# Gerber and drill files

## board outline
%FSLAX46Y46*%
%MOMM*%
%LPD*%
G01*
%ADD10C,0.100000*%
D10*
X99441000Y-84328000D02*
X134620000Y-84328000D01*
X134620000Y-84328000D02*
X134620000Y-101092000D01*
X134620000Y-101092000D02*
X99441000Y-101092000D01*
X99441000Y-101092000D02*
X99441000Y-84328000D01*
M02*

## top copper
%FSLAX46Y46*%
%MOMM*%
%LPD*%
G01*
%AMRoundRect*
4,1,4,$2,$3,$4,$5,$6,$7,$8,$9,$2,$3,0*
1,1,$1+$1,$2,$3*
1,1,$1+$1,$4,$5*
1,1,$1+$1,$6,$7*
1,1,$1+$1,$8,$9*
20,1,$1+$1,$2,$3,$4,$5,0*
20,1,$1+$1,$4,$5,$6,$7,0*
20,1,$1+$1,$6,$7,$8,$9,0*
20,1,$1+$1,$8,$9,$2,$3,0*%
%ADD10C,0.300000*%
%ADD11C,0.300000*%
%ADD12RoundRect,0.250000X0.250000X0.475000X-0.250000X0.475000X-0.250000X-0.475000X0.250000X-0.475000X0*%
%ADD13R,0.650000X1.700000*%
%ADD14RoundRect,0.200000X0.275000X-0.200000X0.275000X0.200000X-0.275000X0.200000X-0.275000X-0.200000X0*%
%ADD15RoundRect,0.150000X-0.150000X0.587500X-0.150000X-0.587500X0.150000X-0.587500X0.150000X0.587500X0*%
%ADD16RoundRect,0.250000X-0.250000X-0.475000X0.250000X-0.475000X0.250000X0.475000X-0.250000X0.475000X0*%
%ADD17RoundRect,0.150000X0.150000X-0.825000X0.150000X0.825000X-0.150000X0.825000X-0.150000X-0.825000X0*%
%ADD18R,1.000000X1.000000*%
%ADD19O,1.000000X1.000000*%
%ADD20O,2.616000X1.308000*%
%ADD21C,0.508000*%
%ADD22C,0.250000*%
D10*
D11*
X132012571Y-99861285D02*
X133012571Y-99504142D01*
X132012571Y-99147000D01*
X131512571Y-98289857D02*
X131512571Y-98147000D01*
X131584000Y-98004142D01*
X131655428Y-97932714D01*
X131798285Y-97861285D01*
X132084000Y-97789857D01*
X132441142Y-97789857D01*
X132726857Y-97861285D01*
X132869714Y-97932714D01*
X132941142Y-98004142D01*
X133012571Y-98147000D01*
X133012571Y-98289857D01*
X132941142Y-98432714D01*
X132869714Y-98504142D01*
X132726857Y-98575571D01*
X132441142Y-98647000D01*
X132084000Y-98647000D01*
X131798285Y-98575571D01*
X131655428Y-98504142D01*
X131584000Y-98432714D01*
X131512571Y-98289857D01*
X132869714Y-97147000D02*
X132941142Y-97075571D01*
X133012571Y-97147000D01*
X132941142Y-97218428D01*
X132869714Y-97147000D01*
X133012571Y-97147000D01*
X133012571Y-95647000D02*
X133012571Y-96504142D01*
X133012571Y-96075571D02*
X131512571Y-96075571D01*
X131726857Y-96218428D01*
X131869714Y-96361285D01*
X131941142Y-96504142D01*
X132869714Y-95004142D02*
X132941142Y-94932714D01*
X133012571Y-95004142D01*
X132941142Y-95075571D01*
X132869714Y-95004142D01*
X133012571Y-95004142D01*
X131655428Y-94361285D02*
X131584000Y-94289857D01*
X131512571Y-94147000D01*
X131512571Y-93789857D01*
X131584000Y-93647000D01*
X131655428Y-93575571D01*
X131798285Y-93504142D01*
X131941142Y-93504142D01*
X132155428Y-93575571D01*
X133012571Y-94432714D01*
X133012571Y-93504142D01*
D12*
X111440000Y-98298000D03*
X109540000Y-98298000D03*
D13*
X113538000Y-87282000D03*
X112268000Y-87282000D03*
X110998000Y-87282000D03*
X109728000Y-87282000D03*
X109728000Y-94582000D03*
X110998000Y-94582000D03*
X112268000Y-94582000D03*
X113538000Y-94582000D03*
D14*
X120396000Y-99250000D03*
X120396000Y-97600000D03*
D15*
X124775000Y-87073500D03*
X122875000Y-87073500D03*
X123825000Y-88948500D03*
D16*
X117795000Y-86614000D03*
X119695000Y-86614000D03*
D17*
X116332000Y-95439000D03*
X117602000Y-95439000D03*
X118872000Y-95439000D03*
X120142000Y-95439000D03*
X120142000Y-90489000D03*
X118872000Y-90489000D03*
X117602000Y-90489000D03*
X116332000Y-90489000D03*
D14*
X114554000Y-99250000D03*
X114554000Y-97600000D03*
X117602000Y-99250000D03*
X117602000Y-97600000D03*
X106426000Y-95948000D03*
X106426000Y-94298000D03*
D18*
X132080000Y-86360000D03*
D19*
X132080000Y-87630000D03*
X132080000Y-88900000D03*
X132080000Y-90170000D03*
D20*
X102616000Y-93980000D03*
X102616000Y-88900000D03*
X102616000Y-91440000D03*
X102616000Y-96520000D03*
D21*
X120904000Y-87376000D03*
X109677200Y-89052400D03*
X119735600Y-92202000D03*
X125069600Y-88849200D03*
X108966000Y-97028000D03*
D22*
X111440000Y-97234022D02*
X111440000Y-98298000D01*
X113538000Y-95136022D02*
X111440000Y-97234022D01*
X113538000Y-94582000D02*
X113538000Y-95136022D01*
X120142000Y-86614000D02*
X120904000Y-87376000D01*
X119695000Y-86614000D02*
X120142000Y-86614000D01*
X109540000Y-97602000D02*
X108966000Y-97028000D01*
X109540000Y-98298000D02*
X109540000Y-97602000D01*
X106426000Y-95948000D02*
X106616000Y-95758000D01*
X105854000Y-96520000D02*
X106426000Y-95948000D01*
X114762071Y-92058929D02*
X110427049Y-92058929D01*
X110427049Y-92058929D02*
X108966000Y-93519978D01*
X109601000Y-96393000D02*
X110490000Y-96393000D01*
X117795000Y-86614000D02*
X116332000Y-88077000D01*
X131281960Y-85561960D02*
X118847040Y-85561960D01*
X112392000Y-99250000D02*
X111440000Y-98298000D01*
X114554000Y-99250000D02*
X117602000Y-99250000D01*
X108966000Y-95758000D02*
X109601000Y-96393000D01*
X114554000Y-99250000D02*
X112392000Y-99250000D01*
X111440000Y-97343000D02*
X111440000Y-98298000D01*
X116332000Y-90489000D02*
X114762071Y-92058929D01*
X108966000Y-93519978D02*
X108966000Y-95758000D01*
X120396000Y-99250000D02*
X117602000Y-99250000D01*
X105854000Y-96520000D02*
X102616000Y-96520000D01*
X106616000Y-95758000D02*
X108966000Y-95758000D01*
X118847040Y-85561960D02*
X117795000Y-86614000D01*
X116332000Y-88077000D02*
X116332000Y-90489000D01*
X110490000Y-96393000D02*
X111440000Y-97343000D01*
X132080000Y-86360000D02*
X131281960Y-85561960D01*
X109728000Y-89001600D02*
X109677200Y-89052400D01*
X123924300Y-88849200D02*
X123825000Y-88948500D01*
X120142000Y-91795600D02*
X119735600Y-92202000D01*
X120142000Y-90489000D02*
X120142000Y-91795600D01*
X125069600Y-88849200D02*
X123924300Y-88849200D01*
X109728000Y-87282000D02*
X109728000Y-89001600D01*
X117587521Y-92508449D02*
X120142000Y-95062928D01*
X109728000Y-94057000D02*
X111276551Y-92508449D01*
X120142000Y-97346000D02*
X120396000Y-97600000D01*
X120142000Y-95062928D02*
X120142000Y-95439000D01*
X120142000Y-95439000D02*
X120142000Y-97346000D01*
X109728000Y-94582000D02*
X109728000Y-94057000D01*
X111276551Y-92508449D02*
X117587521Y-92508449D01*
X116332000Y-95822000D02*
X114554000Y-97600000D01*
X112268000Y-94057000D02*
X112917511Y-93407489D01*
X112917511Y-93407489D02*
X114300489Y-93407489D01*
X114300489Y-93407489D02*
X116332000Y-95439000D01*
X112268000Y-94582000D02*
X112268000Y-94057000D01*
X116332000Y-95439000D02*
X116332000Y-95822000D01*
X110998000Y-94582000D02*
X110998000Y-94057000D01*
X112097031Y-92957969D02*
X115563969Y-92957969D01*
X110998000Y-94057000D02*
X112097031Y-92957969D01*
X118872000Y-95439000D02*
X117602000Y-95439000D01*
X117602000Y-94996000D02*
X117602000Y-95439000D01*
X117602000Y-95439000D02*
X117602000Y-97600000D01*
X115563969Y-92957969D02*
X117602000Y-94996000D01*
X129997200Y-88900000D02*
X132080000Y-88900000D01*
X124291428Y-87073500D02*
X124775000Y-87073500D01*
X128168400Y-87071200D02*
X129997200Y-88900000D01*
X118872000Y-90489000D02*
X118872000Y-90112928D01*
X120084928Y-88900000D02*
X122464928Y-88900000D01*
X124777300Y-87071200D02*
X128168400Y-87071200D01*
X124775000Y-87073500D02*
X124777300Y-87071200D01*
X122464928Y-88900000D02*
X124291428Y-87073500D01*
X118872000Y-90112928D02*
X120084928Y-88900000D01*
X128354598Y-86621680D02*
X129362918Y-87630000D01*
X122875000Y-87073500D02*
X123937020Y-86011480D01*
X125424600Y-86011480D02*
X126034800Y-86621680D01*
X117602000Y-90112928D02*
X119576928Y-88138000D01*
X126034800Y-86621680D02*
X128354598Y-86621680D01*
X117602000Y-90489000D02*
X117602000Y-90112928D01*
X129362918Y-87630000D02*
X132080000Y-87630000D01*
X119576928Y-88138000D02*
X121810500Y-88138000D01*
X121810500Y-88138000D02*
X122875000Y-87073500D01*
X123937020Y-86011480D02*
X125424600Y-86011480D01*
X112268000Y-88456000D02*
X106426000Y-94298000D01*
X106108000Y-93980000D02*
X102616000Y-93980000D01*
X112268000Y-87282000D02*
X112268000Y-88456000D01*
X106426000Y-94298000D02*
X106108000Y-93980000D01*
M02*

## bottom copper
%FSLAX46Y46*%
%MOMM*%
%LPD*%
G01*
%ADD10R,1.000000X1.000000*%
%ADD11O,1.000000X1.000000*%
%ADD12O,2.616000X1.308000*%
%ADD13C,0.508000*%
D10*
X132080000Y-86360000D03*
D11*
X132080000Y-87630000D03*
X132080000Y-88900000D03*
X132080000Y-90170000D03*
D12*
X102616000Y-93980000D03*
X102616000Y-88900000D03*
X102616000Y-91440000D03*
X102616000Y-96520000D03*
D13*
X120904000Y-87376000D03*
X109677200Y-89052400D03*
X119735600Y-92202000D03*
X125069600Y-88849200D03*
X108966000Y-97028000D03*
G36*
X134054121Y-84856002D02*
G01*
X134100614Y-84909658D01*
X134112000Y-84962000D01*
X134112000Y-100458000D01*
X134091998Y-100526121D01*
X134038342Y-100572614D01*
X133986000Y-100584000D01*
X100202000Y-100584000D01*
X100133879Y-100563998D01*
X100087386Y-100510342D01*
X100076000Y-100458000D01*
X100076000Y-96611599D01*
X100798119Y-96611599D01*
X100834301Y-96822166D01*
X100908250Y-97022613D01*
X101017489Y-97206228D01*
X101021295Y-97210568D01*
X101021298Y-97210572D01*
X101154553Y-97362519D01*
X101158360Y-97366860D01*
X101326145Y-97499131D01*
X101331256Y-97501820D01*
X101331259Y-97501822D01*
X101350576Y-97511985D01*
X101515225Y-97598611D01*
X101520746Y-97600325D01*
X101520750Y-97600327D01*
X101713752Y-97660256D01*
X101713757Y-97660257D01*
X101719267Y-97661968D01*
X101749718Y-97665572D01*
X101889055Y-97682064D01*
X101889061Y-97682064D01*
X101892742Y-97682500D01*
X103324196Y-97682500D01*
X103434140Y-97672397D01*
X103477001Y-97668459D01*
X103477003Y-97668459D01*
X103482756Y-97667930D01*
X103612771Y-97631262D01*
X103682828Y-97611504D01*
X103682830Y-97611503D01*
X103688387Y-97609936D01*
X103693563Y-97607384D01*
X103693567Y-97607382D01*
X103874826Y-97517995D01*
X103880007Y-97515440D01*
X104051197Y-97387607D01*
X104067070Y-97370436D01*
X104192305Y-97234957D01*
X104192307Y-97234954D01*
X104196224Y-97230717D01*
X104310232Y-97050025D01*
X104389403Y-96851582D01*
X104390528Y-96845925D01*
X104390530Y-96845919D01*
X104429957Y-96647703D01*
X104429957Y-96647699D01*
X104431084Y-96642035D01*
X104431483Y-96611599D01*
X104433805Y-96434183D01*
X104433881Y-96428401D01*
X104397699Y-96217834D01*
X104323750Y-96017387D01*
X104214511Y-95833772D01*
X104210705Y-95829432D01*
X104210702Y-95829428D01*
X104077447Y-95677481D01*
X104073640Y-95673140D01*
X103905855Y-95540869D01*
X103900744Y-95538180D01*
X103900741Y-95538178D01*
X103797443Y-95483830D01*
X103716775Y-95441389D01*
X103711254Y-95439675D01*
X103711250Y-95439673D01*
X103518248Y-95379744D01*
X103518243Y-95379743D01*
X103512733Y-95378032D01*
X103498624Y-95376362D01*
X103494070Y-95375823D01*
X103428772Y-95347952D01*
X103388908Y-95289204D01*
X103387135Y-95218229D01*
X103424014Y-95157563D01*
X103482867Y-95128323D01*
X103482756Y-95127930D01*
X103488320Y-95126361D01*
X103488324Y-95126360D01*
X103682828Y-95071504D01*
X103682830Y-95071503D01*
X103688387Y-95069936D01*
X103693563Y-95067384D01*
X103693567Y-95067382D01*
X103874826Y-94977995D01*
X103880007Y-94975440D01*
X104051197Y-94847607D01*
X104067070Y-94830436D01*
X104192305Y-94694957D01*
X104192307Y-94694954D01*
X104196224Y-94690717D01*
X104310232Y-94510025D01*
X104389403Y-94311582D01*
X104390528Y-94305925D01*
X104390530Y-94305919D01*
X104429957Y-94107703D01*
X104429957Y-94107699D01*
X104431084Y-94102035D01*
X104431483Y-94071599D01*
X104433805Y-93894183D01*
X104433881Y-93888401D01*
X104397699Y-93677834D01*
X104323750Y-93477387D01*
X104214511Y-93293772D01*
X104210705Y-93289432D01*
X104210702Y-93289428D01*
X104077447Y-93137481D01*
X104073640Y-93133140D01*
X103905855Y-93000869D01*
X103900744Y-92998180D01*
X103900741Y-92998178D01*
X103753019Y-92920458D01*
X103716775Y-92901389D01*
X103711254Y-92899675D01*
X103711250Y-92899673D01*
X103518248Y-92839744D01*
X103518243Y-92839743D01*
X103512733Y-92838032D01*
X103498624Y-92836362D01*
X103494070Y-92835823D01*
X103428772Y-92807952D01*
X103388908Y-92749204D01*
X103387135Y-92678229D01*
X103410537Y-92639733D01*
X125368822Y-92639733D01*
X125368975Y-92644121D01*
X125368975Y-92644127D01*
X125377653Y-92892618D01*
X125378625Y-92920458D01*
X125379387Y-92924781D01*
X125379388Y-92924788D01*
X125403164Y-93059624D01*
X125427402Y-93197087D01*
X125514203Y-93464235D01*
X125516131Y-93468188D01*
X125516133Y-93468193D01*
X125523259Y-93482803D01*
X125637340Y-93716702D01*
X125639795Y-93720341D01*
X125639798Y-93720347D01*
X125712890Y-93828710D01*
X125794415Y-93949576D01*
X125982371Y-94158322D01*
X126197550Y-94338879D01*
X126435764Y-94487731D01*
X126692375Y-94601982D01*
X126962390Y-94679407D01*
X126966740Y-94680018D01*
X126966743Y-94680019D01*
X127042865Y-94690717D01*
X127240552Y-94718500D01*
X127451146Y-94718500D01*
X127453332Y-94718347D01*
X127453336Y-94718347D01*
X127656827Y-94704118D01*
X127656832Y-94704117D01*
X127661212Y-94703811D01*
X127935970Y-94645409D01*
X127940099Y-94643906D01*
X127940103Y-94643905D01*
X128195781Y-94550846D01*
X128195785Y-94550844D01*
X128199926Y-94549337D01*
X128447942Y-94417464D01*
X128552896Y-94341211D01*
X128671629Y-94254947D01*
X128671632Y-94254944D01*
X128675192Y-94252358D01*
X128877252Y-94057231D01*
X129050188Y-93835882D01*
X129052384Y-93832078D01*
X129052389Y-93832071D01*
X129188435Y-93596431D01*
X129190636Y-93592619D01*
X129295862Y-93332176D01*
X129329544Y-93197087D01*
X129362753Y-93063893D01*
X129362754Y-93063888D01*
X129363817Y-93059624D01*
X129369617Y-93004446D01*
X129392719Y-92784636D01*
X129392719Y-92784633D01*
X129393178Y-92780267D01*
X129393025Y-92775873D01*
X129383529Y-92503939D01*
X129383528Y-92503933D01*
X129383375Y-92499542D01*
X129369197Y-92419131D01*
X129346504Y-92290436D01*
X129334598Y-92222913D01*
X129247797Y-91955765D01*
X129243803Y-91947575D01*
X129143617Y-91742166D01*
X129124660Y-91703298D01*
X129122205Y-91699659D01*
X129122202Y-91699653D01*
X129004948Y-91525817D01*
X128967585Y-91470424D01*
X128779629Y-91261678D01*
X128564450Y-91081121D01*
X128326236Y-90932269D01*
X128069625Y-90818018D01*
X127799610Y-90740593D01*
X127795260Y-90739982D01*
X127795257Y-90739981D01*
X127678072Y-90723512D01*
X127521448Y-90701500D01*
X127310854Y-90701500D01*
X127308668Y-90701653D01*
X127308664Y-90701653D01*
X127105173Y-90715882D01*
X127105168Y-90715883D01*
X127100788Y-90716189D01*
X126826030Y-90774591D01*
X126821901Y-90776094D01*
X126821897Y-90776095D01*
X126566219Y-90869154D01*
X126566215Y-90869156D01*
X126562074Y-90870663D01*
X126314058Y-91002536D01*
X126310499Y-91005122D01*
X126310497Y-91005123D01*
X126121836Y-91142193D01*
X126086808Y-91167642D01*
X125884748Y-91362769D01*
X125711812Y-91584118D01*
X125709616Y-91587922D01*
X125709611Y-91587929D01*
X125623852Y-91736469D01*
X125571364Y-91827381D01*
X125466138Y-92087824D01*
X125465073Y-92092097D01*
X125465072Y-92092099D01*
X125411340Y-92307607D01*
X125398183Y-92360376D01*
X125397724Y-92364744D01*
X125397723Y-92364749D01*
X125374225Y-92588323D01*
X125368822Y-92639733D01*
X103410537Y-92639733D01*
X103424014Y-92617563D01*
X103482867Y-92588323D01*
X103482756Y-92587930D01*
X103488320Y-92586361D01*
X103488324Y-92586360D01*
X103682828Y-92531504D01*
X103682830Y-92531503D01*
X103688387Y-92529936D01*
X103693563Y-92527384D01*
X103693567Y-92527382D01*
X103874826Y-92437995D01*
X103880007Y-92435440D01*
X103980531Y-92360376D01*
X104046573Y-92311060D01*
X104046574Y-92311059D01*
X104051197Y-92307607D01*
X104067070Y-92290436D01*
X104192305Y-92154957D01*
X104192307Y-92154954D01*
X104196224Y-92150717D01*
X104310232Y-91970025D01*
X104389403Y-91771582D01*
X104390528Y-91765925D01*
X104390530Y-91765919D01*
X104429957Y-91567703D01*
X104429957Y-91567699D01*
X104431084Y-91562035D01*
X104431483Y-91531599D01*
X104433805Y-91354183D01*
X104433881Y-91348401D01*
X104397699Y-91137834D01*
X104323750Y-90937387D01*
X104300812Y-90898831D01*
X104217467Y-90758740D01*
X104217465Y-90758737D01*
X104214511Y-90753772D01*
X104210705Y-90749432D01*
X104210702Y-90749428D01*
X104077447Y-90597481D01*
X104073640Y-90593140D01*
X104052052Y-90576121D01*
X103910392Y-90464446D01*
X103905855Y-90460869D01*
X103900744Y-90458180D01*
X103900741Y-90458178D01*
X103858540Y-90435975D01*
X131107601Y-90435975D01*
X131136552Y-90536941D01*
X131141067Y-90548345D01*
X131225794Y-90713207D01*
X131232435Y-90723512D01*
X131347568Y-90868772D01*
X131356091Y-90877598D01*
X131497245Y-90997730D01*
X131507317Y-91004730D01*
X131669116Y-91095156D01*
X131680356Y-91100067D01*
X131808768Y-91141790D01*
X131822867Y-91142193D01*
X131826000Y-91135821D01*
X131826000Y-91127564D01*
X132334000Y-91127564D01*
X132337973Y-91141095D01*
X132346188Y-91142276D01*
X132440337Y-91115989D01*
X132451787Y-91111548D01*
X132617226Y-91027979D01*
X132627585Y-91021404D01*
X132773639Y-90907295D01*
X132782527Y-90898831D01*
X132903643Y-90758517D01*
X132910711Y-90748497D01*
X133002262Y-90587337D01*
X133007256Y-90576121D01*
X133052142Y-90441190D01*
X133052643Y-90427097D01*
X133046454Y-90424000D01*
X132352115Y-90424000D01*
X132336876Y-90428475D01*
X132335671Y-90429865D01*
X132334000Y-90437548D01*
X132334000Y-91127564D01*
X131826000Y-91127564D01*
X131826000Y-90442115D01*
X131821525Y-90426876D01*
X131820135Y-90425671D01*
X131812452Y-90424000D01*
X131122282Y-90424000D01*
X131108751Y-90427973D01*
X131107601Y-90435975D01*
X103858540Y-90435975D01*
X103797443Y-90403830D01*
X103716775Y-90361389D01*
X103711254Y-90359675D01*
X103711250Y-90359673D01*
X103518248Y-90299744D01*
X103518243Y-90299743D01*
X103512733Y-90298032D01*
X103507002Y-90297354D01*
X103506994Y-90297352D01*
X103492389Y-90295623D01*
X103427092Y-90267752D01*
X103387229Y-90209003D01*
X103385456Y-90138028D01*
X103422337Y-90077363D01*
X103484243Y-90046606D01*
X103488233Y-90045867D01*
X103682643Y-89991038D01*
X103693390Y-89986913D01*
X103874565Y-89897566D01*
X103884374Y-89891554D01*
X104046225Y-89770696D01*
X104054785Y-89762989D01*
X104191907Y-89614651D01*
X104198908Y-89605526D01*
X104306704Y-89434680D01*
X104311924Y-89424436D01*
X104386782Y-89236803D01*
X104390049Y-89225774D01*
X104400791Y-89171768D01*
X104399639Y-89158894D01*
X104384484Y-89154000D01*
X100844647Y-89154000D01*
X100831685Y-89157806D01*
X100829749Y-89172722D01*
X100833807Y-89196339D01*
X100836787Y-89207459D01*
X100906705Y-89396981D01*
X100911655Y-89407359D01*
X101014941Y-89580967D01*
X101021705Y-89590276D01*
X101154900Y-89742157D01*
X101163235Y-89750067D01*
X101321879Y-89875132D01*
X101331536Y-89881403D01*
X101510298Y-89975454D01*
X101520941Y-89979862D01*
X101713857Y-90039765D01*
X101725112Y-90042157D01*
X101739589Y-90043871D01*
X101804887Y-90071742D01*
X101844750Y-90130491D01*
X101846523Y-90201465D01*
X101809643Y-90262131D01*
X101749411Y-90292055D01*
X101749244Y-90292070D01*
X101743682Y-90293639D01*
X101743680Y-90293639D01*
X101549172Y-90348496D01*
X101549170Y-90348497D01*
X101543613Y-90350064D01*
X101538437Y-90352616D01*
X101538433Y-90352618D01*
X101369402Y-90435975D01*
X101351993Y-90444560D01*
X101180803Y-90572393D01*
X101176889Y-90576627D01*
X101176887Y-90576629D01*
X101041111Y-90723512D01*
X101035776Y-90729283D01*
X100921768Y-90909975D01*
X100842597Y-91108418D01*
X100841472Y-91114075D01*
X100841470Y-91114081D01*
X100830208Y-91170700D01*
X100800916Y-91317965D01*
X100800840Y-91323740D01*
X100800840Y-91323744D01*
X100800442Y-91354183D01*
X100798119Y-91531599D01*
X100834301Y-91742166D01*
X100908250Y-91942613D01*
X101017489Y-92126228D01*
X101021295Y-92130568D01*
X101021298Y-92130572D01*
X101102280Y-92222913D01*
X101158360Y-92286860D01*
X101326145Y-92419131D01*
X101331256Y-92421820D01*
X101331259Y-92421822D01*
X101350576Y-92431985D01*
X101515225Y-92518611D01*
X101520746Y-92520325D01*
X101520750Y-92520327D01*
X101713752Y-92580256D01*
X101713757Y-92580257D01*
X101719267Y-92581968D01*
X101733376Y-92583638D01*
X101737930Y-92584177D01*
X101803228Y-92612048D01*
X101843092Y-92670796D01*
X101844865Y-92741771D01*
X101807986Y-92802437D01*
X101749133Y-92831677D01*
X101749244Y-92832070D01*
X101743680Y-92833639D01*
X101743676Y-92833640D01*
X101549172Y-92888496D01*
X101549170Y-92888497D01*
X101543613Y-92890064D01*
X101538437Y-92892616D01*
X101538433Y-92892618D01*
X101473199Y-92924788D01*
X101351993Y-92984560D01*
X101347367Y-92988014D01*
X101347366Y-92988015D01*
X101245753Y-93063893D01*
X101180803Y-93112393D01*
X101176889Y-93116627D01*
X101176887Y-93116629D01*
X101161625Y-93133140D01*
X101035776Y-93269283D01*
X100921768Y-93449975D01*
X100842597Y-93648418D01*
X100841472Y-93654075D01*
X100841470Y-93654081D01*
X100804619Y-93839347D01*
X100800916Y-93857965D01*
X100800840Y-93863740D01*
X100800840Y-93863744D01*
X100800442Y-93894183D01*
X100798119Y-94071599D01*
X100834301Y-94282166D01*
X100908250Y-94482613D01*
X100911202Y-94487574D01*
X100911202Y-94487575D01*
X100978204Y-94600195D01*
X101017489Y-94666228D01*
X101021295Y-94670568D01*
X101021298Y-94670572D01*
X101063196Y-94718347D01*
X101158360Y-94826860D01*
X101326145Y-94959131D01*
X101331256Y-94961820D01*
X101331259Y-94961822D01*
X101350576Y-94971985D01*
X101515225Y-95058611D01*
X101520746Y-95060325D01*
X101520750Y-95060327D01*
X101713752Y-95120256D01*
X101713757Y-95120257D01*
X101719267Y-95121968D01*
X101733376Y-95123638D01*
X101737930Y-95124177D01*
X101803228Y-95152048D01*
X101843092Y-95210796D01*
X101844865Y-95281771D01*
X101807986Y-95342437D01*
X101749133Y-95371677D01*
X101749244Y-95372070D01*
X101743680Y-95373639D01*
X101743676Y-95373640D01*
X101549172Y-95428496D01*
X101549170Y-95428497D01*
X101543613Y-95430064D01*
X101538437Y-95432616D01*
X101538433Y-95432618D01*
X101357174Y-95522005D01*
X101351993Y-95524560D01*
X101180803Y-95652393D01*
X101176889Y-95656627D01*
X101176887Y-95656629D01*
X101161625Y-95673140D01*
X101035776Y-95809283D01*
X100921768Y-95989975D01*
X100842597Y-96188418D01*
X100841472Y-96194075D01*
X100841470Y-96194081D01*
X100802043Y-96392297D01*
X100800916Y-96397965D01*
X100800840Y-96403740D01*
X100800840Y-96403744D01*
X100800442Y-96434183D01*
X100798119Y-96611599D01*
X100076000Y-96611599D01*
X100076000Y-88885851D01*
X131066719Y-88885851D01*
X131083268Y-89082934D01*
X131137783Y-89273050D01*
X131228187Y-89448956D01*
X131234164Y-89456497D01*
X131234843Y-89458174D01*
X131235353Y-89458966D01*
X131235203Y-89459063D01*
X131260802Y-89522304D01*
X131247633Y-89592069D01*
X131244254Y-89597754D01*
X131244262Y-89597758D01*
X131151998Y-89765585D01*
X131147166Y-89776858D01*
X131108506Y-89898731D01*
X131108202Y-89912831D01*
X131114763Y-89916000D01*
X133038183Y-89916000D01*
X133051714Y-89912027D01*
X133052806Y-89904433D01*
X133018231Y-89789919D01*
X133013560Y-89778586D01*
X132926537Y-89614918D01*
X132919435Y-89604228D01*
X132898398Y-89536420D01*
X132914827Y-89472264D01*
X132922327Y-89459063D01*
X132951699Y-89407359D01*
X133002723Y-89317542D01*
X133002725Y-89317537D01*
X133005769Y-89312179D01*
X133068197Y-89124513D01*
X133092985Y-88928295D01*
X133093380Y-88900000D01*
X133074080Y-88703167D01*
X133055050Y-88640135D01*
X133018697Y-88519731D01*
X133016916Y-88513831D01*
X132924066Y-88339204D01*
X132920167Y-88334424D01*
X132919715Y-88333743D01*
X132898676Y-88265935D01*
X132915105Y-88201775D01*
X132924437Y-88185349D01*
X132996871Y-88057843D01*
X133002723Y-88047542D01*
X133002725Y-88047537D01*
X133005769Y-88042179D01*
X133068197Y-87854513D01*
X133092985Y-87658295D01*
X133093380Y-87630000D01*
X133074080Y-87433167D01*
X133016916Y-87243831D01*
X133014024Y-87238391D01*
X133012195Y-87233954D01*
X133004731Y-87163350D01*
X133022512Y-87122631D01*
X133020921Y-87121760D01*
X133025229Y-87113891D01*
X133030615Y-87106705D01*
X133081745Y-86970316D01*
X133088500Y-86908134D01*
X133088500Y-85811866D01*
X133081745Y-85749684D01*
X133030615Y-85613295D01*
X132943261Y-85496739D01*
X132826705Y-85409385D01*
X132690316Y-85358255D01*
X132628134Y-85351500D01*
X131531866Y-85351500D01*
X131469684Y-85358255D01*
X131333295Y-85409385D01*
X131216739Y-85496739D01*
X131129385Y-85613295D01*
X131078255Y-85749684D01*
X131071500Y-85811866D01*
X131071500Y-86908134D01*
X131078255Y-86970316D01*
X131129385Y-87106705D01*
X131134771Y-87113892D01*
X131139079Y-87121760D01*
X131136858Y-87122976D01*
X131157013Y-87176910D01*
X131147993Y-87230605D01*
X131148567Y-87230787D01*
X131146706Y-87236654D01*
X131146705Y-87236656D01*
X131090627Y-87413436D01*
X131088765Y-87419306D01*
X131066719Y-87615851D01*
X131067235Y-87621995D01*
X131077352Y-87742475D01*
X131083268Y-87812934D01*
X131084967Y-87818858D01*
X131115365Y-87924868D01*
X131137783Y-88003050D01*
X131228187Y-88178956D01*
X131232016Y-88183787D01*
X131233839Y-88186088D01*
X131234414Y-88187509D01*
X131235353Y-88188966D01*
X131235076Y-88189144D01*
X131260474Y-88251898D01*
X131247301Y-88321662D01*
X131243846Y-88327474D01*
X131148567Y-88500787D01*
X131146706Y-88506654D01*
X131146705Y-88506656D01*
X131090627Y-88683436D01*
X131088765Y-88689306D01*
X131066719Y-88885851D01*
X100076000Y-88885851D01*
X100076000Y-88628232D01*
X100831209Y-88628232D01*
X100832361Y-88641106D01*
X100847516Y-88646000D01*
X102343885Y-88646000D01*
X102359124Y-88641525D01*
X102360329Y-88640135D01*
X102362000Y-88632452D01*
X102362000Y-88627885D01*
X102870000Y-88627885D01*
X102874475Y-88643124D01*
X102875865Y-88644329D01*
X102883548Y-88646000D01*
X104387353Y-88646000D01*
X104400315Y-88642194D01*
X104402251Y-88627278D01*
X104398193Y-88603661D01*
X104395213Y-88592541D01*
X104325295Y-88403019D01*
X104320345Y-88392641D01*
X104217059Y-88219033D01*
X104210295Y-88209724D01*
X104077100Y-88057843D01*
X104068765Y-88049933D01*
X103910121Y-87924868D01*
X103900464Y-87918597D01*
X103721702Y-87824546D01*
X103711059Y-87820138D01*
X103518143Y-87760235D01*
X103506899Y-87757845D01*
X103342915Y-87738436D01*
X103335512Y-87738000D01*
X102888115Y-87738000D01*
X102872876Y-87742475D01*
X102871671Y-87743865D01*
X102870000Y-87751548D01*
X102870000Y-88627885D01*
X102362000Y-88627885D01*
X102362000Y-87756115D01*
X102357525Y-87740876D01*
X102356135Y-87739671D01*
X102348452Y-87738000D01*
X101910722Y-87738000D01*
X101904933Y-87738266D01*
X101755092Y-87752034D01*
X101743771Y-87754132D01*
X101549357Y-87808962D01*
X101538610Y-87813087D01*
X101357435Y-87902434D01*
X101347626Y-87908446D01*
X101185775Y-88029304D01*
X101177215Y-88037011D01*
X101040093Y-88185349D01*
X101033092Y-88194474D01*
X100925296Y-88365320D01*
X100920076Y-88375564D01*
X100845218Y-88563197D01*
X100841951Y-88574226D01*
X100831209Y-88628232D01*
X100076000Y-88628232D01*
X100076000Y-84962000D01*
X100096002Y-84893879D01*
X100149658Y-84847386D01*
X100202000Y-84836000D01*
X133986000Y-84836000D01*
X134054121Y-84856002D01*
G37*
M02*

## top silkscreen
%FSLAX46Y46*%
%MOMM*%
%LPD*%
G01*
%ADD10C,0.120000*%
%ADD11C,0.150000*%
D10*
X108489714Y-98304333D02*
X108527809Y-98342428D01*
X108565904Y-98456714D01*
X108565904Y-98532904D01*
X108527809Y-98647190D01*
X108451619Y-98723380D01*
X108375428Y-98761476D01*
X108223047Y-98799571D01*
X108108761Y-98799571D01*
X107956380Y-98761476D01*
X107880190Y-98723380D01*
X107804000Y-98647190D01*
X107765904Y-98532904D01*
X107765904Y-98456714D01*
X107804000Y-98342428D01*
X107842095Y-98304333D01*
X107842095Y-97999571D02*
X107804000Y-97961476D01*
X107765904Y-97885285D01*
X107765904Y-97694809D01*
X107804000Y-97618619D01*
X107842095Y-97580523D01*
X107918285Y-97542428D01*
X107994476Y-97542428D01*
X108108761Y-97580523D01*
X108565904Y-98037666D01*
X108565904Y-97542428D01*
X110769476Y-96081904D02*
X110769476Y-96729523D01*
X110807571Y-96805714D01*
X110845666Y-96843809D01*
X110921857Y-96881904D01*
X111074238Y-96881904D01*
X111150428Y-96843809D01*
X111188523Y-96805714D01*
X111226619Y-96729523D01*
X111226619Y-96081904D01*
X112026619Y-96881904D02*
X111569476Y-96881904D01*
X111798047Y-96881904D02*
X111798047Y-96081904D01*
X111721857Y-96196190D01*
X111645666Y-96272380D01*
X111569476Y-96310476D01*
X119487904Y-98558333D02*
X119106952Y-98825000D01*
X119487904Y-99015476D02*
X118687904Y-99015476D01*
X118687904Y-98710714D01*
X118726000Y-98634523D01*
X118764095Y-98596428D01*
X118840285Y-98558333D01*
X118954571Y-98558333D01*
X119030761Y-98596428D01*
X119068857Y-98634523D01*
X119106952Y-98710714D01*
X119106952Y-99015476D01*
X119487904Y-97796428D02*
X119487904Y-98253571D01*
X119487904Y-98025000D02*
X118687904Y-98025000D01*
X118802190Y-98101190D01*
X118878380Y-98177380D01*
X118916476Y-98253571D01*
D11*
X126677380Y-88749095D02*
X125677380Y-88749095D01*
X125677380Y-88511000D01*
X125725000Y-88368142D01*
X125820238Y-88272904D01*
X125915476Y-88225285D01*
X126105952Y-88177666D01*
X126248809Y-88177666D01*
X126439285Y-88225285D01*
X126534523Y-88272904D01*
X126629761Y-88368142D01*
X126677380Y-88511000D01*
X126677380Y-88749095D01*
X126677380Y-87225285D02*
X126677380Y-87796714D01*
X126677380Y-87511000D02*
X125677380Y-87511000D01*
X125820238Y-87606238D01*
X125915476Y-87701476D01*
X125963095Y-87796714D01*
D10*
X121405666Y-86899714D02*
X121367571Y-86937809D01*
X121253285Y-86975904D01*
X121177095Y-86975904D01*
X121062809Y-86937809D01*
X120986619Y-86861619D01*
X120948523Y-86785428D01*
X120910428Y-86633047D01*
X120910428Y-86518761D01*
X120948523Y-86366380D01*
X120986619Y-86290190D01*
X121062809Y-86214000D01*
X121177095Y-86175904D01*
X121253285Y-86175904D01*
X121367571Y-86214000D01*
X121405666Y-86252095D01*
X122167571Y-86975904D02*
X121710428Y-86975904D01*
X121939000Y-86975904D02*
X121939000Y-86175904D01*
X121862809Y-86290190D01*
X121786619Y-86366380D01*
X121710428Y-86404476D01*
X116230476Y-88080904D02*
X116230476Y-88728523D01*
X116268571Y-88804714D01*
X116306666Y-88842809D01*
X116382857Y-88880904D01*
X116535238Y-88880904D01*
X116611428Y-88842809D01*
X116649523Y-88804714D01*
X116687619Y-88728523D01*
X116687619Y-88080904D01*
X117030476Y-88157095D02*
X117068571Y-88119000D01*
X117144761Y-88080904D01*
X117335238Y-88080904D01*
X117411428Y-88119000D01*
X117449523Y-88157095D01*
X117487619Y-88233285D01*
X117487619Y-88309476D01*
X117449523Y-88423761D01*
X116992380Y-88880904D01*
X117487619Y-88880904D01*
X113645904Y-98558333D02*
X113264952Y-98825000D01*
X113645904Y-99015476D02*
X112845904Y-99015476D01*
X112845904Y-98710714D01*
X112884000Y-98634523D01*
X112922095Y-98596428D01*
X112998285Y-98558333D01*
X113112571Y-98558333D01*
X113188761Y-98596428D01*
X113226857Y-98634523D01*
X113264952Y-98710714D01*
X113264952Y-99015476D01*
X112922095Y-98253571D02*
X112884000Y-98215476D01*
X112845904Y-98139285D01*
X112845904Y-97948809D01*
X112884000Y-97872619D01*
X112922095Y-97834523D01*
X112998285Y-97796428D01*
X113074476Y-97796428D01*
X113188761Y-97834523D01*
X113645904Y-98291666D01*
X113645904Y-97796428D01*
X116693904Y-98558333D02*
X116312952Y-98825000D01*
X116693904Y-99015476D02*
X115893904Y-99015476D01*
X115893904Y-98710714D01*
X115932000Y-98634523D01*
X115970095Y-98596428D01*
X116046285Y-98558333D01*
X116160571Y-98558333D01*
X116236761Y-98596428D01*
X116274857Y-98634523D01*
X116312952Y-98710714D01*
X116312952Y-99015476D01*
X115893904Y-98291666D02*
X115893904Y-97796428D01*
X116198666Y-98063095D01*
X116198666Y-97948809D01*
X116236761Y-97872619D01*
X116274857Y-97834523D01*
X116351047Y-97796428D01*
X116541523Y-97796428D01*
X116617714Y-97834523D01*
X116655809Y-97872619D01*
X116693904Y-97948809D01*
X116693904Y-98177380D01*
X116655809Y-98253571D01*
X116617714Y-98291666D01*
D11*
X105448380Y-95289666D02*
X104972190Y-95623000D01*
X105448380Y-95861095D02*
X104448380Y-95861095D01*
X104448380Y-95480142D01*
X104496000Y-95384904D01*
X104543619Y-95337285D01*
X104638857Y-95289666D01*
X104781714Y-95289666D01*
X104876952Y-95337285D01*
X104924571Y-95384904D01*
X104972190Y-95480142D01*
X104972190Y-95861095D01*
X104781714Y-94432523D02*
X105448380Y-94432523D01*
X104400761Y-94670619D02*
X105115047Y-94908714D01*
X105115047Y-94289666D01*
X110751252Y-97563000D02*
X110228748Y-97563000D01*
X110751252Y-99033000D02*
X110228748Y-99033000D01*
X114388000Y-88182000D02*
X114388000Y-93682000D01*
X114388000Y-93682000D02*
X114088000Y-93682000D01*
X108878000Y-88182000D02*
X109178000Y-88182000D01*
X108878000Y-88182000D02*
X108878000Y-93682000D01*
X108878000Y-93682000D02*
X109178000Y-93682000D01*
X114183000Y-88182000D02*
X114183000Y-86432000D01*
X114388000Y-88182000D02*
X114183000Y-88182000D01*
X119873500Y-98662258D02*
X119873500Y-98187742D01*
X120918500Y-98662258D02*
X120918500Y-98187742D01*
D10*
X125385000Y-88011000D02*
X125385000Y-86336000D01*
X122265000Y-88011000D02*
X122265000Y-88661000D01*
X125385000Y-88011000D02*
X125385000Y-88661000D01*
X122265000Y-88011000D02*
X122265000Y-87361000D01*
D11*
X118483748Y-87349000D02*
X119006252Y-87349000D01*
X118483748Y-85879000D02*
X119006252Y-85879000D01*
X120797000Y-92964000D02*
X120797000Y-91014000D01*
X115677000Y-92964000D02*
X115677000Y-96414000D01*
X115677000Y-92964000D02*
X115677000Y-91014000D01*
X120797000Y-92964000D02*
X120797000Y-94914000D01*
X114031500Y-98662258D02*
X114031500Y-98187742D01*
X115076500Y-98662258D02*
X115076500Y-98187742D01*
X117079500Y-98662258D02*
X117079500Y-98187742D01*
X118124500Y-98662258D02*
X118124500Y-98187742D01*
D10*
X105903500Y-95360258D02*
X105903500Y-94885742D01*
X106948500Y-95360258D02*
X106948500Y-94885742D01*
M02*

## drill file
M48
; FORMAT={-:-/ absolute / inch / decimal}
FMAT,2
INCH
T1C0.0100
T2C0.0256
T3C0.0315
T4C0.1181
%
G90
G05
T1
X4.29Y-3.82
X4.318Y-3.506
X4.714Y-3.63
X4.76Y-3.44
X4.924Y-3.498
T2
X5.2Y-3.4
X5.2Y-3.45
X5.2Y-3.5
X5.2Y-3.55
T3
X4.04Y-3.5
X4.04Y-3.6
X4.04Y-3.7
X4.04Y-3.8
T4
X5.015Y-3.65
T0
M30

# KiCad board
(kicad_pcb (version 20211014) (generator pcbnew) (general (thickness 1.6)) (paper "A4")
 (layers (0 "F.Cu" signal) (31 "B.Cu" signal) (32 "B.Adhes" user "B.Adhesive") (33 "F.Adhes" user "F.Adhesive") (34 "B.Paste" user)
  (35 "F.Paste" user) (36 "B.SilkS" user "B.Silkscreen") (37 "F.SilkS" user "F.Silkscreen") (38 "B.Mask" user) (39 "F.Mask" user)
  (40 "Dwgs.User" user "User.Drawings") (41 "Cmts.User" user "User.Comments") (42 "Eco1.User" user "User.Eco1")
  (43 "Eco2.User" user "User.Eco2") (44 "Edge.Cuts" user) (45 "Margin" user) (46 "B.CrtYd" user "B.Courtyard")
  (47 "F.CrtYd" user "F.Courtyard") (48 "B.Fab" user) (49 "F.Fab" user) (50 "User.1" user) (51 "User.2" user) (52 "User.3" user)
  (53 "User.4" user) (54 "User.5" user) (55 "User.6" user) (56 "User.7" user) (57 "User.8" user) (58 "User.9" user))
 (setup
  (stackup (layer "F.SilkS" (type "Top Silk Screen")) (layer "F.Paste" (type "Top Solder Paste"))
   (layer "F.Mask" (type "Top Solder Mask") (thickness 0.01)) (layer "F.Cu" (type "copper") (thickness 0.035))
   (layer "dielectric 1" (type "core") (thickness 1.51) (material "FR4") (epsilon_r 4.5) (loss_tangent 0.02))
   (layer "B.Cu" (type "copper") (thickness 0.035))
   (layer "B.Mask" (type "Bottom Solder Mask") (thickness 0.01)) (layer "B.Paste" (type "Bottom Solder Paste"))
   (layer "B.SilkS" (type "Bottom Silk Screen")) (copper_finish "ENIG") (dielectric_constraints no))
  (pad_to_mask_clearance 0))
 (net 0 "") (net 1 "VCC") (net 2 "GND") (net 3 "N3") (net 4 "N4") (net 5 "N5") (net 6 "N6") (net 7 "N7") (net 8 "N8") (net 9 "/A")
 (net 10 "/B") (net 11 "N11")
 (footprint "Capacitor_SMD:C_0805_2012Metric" (layer "F.Cu") (at 110.49 98.298 180)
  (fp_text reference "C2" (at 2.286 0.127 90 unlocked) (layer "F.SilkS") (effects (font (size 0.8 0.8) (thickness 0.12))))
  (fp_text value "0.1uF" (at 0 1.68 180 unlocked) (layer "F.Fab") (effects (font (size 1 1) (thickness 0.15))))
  (fp_line (start -0.261252 0.735) (end 0.261252 0.735) (layer "F.SilkS") (width 0.15))
  (fp_line (start -0.261252 -0.735) (end 0.261252 -0.735) (layer "F.SilkS") (width 0.15))
  (pad "1" smd roundrect locked (at -0.95 0 180) (size 1 1.45) (layers "F.Cu" "F.Paste" "F.Mask") (roundrect_rratio 0.25) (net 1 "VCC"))
  (pad "2" smd roundrect locked (at 0.95 0 180) (size 1 1.45) (layers "F.Cu" "F.Paste" "F.Mask") (roundrect_rratio 0.25) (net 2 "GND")))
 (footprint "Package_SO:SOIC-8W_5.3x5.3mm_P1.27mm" (layer "F.Cu") (at 111.633 90.932 -90)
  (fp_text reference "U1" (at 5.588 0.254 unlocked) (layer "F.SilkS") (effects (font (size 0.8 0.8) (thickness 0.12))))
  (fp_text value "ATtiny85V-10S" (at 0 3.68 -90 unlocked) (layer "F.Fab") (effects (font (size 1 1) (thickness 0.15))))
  (fp_line (start -2.75 -2.755) (end 2.75 -2.755) (layer "F.SilkS") (width 0.15))
  (fp_line (start 2.75 -2.755) (end 2.75 -2.455) (layer "F.SilkS") (width 0.15))
  (fp_line (start -2.75 2.755) (end -2.75 2.455) (layer "F.SilkS") (width 0.15))
  (fp_line (start -2.75 2.755) (end 2.75 2.755) (layer "F.SilkS") (width 0.15))
  (fp_line (start 2.75 2.755) (end 2.75 2.455) (layer "F.SilkS") (width 0.15))
  (fp_line (start -2.75 -2.55) (end -4.5 -2.55) (layer "F.SilkS") (width 0.15))
  (fp_line (start -2.75 -2.755) (end -2.75 -2.55) (layer "F.SilkS") (width 0.15))
  (pad "1" smd rect locked (at -3.65 -1.905 270) (size 1.7 0.65) (layers "F.Cu" "F.Paste" "F.Mask") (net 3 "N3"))
  (pad "2" smd rect locked (at -3.65 -0.635 270) (size 1.7 0.65) (layers "F.Cu" "F.Paste" "F.Mask") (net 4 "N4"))
  (pad "3" smd rect locked (at -3.65 0.635 270) (size 1.7 0.65) (layers "F.Cu" "F.Paste" "F.Mask") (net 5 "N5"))
  (pad "4" smd rect locked (at -3.65 1.905 270) (size 1.7 0.65) (layers "F.Cu" "F.Paste" "F.Mask") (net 2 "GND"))
  (pad "5" smd rect locked (at 3.65 1.905 270) (size 1.7 0.65) (layers "F.Cu" "F.Paste" "F.Mask") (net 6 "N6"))
  (pad "6" smd rect locked (at 3.65 0.635 270) (size 1.7 0.65) (layers "F.Cu" "F.Paste" "F.Mask") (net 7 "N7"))
  (pad "7" smd rect locked (at 3.65 -0.635 270) (size 1.7 0.65) (layers "F.Cu" "F.Paste" "F.Mask") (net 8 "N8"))
  (pad "8" smd rect locked (at 3.65 -1.905 270) (size 1.7 0.65) (layers "F.Cu" "F.Paste" "F.Mask") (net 1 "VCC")))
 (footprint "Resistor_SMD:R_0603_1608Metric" (layer "F.Cu") (at 120.396 98.425 90)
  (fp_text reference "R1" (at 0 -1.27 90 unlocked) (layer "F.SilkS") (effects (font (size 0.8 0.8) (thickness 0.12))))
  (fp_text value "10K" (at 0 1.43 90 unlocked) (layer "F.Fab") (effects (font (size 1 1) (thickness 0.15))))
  (fp_line (start -0.237258 -0.5225) (end 0.237258 -0.5225) (layer "F.SilkS") (width 0.15))
  (fp_line (start -0.237258 0.5225) (end 0.237258 0.5225) (layer "F.SilkS") (width 0.15))
  (pad "1" smd roundrect locked (at -0.825 0 90) (size 0.8 0.95) (layers "F.Cu" "F.Paste" "F.Mask") (roundrect_rratio 0.25) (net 1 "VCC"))
  (pad "2" smd roundrect locked (at 0.825 0 90) (size 0.8 0.95) (layers "F.Cu" "F.Paste" "F.Mask") (roundrect_rratio 0.25) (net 6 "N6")))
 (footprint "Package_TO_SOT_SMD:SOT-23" (layer "F.Cu") (at 123.825 88.011 -90)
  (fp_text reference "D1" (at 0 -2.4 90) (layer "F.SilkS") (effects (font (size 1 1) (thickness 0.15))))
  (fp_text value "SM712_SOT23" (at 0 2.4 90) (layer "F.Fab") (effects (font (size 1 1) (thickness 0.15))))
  (fp_line (start 0 -1.56) (end -1.675 -1.56) (layer "F.SilkS") (width 0.12))
  (fp_line (start 0 1.56) (end 0.65 1.56) (layer "F.SilkS") (width 0.12))
  (fp_line (start 0 -1.56) (end 0.65 -1.56) (layer "F.SilkS") (width 0.12))
  (fp_line (start 0 1.56) (end -0.65 1.56) (layer "F.SilkS") (width 0.12))
  (pad "1" smd roundrect locked (at -0.9375 -0.95 270) (size 1.475 0.6) (layers "F.Cu" "F.Paste" "F.Mask") (roundrect_rratio 0.25)
   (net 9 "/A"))
  (pad "2" smd roundrect locked (at -0.9375 0.95 270) (size 1.475 0.6) (layers "F.Cu" "F.Paste" "F.Mask") (roundrect_rratio 0.25)
   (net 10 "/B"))
  (pad "3" smd roundrect locked (at 0.9375 0 270) (size 1.475 0.6) (layers "F.Cu" "F.Paste" "F.Mask") (roundrect_rratio 0.25) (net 2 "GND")))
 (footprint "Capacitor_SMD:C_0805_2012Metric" (layer "F.Cu") (at 118.745 86.614)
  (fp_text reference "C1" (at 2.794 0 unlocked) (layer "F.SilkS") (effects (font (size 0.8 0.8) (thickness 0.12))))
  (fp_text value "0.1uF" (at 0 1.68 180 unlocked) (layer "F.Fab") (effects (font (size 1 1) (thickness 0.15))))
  (fp_line (start -0.261252 0.735) (end 0.261252 0.735) (layer "F.SilkS") (width 0.15))
  (fp_line (start -0.261252 -0.735) (end 0.261252 -0.735) (layer "F.SilkS") (width 0.15))
  (pad "1" smd roundrect locked (at -0.95 0) (size 1 1.45) (layers "F.Cu" "F.Paste" "F.Mask") (roundrect_rratio 0.25) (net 1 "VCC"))
  (pad "2" smd roundrect locked (at 0.95 0) (size 1 1.45) (layers "F.Cu" "F.Paste" "F.Mask") (roundrect_rratio 0.25) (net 2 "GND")))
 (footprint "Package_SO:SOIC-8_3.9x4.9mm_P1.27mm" (layer "F.Cu") (at 118.237 92.964 90)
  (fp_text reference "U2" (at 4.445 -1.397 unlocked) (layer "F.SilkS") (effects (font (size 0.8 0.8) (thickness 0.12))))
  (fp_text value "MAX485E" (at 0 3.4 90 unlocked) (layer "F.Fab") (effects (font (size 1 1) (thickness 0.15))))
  (fp_line (start 0 2.56) (end 1.95 2.56) (layer "F.SilkS") (width 0.15))
  (fp_line (start 0 -2.56) (end -3.45 -2.56) (layer "F.SilkS") (width 0.15))
  (fp_line (start 0 -2.56) (end 1.95 -2.56) (layer "F.SilkS") (width 0.15))
  (fp_line (start 0 2.56) (end -1.95 2.56) (layer "F.SilkS") (width 0.15))
  (pad "1" smd roundrect locked (at -2.475 -1.905 90) (size 1.95 0.6) (layers "F.Cu" "F.Paste" "F.Mask") (roundrect_rratio 0.25)
   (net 8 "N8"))
  (pad "2" smd roundrect locked (at -2.475 -0.635 90) (size 1.95 0.6) (layers "F.Cu" "F.Paste" "F.Mask") (roundrect_rratio 0.25)
   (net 7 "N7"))
  (pad "3" smd roundrect locked (at -2.475 0.635 90) (size 1.95 0.6) (layers "F.Cu" "F.Paste" "F.Mask") (roundrect_rratio 0.25) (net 7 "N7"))
  (pad "4" smd roundrect locked (at -2.475 1.905 90) (size 1.95 0.6) (layers "F.Cu" "F.Paste" "F.Mask") (roundrect_rratio 0.25) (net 6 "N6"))
  (pad "5" smd roundrect locked (at 2.475 1.905 90) (size 1.95 0.6) (layers "F.Cu" "F.Paste" "F.Mask") (roundrect_rratio 0.25) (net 2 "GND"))
  (pad "6" smd roundrect locked (at 2.475 0.635 90) (size 1.95 0.6) (layers "F.Cu" "F.Paste" "F.Mask") (roundrect_rratio 0.25) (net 9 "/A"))
  (pad "7" smd roundrect locked (at 2.475 -0.635 90) (size 1.95 0.6) (layers "F.Cu" "F.Paste" "F.Mask") (roundrect_rratio 0.25)
   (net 10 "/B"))
  (pad "8" smd roundrect locked (at 2.475 -1.905 90) (size 1.95 0.6) (layers "F.Cu" "F.Paste" "F.Mask") (roundrect_rratio 0.25)
   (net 1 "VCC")))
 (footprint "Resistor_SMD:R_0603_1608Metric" (layer "F.Cu") (at 114.554 98.425 90)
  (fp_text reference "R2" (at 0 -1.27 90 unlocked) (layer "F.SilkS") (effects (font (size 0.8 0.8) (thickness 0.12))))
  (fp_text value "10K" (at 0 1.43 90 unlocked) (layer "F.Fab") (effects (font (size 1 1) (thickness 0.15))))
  (fp_line (start -0.237258 -0.5225) (end 0.237258 -0.5225) (layer "F.SilkS") (width 0.15))
  (fp_line (start -0.237258 0.5225) (end 0.237258 0.5225) (layer "F.SilkS") (width 0.15))
  (pad "1" smd roundrect locked (at -0.825 0 90) (size 0.8 0.95) (layers "F.Cu" "F.Paste" "F.Mask") (roundrect_rratio 0.25) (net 1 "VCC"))
  (pad "2" smd roundrect locked (at 0.825 0 90) (size 0.8 0.95) (layers "F.Cu" "F.Paste" "F.Mask") (roundrect_rratio 0.25) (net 8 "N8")))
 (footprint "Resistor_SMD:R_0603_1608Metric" (layer "F.Cu") (at 117.602 98.425 90)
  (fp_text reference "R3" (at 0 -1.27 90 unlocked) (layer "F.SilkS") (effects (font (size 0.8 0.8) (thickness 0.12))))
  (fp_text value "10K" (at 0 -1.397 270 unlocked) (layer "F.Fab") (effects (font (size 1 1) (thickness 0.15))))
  (fp_line (start -0.237258 -0.5225) (end 0.237258 -0.5225) (layer "F.SilkS") (width 0.15))
  (fp_line (start -0.237258 0.5225) (end 0.237258 0.5225) (layer "F.SilkS") (width 0.15))
  (pad "1" smd roundrect locked (at -0.825 0 90) (size 0.8 0.95) (layers "F.Cu" "F.Paste" "F.Mask") (roundrect_rratio 0.25) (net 1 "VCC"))
  (pad "2" smd roundrect locked (at 0.825 0 90) (size 0.8 0.95) (layers "F.Cu" "F.Paste" "F.Mask") (roundrect_rratio 0.25) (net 7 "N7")))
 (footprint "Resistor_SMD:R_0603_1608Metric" (layer "F.Cu") (at 106.426 95.123 90)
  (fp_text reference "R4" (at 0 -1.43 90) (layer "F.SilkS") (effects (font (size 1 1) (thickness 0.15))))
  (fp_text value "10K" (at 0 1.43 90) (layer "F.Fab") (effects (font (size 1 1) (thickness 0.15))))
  (fp_line (start -0.237258 -0.5225) (end 0.237258 -0.5225) (layer "F.SilkS") (width 0.12))
  (fp_line (start -0.237258 0.5225) (end 0.237258 0.5225) (layer "F.SilkS") (width 0.12))
  (pad "1" smd roundrect locked (at -0.825 0 90) (size 0.8 0.95) (layers "F.Cu" "F.Paste" "F.Mask") (roundrect_rratio 0.25) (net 1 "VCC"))
  (pad "2" smd roundrect locked (at 0.825 0 90) (size 0.8 0.95) (layers "F.Cu" "F.Paste" "F.Mask") (roundrect_rratio 0.25) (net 4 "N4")))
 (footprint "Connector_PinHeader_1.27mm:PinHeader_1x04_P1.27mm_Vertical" (layer "B.Cu") (at 132.08 86.36 180)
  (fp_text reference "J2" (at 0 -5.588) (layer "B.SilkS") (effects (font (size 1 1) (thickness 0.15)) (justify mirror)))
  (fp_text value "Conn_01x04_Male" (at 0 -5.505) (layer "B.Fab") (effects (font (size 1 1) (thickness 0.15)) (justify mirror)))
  (pad "1" thru_hole rect locked (at 0 0 180) (size 1 1) (drill 0.65) (layers *.Cu *.Mask) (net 1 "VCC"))
  (pad "2" thru_hole oval locked (at 0 -1.27 180) (size 1 1) (drill 0.65) (layers *.Cu *.Mask) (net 10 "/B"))
  (pad "3" thru_hole oval locked (at 0 -2.54 180) (size 1 1) (drill 0.65) (layers *.Cu *.Mask) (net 9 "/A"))
  (pad "4" thru_hole oval locked (at 0 -3.81 180) (size 1 1) (drill 0.65) (layers *.Cu *.Mask) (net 2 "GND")))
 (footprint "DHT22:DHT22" (layer "B.Cu") (at 102.616 92.71 90)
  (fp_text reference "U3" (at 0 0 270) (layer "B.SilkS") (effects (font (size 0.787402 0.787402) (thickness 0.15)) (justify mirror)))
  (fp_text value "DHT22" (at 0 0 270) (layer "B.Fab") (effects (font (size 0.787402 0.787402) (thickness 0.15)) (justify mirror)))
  (pad "" np_thru_hole circle locked (at 0 24.765 90) (size 3 3) (drill 3) (layers *.Cu *.Mask))
  (pad "DATA" thru_hole oval locked (at -1.27 0 90) (size 1.308 2.616) (drill 0.8) (layers *.Cu *.Mask) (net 4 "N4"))
  (pad "GND" thru_hole oval locked (at 3.81 0 90) (size 1.308 2.616) (drill 0.8) (layers *.Cu *.Mask) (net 2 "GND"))
  (pad "NC" thru_hole oval locked (at 1.27 0 90) (size 1.308 2.616) (drill 0.8) (layers *.Cu *.Mask) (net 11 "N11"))
  (pad "VDD" thru_hole oval locked (at -3.81 0 90) (size 1.308 2.616) (drill 0.8) (layers *.Cu *.Mask) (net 1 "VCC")))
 (gr_rect (start 99.441 84.328) (end 134.62 101.092) (layer "Edge.Cuts") (width 0.1) (fill none))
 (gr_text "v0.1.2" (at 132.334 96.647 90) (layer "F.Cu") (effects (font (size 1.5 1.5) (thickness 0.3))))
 (segment (start 106.426 95.948) (end 106.616 95.758) (width 0.25) (layer "F.Cu") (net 1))
 (segment (start 111.44 97.234022) (end 111.44 98.298) (width 0.25) (layer "F.Cu") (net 1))
 (segment (start 105.854 96.52) (end 106.426 95.948) (width 0.25) (layer "F.Cu") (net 1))
 (segment (start 114.762071 92.058929) (end 110.427049 92.058929) (width 0.25) (layer "F.Cu") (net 1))
 (segment (start 110.427049 92.058929) (end 108.966 93.519978) (width 0.25) (layer "F.Cu") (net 1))
 (segment (start 113.538 95.136022) (end 111.44 97.234022) (width 0.25) (layer "F.Cu") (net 1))
 (segment (start 109.601 96.393) (end 110.49 96.393) (width 0.25) (layer "F.Cu") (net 1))
 (segment (start 117.795 86.614) (end 116.332 88.077) (width 0.25) (layer "F.Cu") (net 1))
 (segment (start 131.28196 85.56196) (end 118.84704 85.56196) (width 0.25) (layer "F.Cu") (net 1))
 (segment (start 112.392 99.25) (end 111.44 98.298) (width 0.25) (layer "F.Cu") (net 1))
 (segment (start 114.554 99.25) (end 117.602 99.25) (width 0.25) (layer "F.Cu") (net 1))
 (segment (start 108.966 95.758) (end 109.601 96.393) (width 0.25) (layer "F.Cu") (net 1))
 (segment (start 113.538 94.582) (end 113.538 95.136022) (width 0.25) (layer "F.Cu") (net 1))
 (segment (start 114.554 99.25) (end 112.392 99.25) (width 0.25) (layer "F.Cu") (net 1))
 (segment (start 111.44 97.343) (end 111.44 98.298) (width 0.25) (layer "F.Cu") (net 1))
 (segment (start 116.332 90.489) (end 114.762071 92.058929) (width 0.25) (layer "F.Cu") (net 1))
 (segment (start 108.966 93.519978) (end 108.966 95.758) (width 0.25) (layer "F.Cu") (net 1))
 (segment (start 120.396 99.25) (end 117.602 99.25) (width 0.25) (layer "F.Cu") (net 1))
 (segment (start 105.854 96.52) (end 102.616 96.52) (width 0.25) (layer "F.Cu") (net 1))
 (segment (start 106.616 95.758) (end 108.966 95.758) (width 0.25) (layer "F.Cu") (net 1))
 (segment (start 118.84704 85.56196) (end 117.795 86.614) (width 0.25) (layer "F.Cu") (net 1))
 (segment (start 116.332 88.077) (end 116.332 90.489) (width 0.25) (layer "F.Cu") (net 1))
 (segment (start 110.49 96.393) (end 111.44 97.343) (width 0.25) (layer "F.Cu") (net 1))
 (segment (start 132.08 86.36) (end 131.28196 85.56196) (width 0.25) (layer "F.Cu") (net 1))
 (segment (start 109.728 89.0016) (end 109.6772 89.0524) (width 0.25) (layer "F.Cu") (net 2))
 (segment (start 123.9243 88.8492) (end 123.825 88.9485) (width 0.25) (layer "F.Cu") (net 2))
 (segment (start 120.142 91.7956) (end 119.7356 92.202) (width 0.25) (layer "F.Cu") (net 2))
 (segment (start 120.142 86.614) (end 120.904 87.376) (width 0.25) (layer "F.Cu") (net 2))
 (segment (start 109.54 97.602) (end 108.966 97.028) (width 0.25) (layer "F.Cu") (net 2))
 (segment (start 109.54 98.298) (end 109.54 97.602) (width 0.25) (layer "F.Cu") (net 2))
 (segment (start 120.142 90.489) (end 120.142 91.7956) (width 0.25) (layer "F.Cu") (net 2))
 (segment (start 125.0696 88.8492) (end 123.9243 88.8492) (width 0.25) (layer "F.Cu") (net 2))
 (segment (start 119.695 86.614) (end 120.142 86.614) (width 0.25) (layer "F.Cu") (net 2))
 (segment (start 109.728 87.282) (end 109.728 89.0016) (width 0.25) (layer "F.Cu") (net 2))
 (via (at 120.904 87.376) (size 0.508) (drill 0.254) (layers "F.Cu" "B.Cu") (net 2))
 (via (at 109.6772 89.0524) (size 0.508) (drill 0.254) (layers "F.Cu" "B.Cu") (free) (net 2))
 (via (at 119.7356 92.202) (size 0.508) (drill 0.254) (layers "F.Cu" "B.Cu") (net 2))
 (via (at 125.0696 88.8492) (size 0.508) (drill 0.254) (layers "F.Cu" "B.Cu") (free) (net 2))
 (via (at 108.966 97.028) (size 0.508) (drill 0.254) (layers "F.Cu" "B.Cu") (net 2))
 (segment (start 117.587521 92.508449) (end 120.142 95.062928) (width 0.25) (layer "F.Cu") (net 6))
 (segment (start 109.728 94.057) (end 111.276551 92.508449) (width 0.25) (layer "F.Cu") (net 6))
 (segment (start 120.142 97.346) (end 120.396 97.6) (width 0.25) (layer "F.Cu") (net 6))
 (segment (start 120.142 95.062928) (end 120.142 95.439) (width 0.25) (layer "F.Cu") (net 6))
 (segment (start 120.142 95.439) (end 120.142 97.346) (width 0.25) (layer "F.Cu") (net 6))
 (segment (start 109.728 94.582) (end 109.728 94.057) (width 0.25) (layer "F.Cu") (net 6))
 (segment (start 111.276551 92.508449) (end 117.587521 92.508449) (width 0.25) (layer "F.Cu") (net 6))
 (segment (start 116.332 95.822) (end 114.554 97.6) (width 0.25) (layer "F.Cu") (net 8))
 (segment (start 112.268 94.057) (end 112.917511 93.407489) (width 0.25) (layer "F.Cu") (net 8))
 (segment (start 112.917511 93.407489) (end 114.300489 93.407489) (width 0.25) (layer "F.Cu") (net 8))
 (segment (start 114.300489 93.407489) (end 116.332 95.439) (width 0.25) (layer "F.Cu") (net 8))
 (segment (start 112.268 94.582) (end 112.268 94.057) (width 0.25) (layer "F.Cu") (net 8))
 (segment (start 116.332 95.439) (end 116.332 95.822) (width 0.25) (layer "F.Cu") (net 8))
 (segment (start 110.998 94.582) (end 110.998 94.057) (width 0.25) (layer "F.Cu") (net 7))
 (segment (start 112.097031 92.957969) (end 115.563969 92.957969) (width 0.25) (layer "F.Cu") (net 7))
 (segment (start 110.998 94.057) (end 112.097031 92.957969) (width 0.25) (layer "F.Cu") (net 7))
 (segment (start 118.872 95.439) (end 117.602 95.439) (width 0.25) (layer "F.Cu") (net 7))
 (segment (start 117.602 94.996) (end 117.602 95.439) (width 0.25) (layer "F.Cu") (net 7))
 (segment (start 117.602 95.439) (end 117.602 97.6) (width 0.25) (layer "F.Cu") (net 7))
 (segment (start 115.563969 92.957969) (end 117.602 94.996) (width 0.25) (layer "F.Cu") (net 7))
 (segment (start 129.9972 88.9) (end 132.08 88.9) (width 0.25) (layer "F.Cu") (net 9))
 (segment (start 124.291428 87.0735) (end 124.775 87.0735) (width 0.25) (layer "F.Cu") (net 9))
 (segment (start 128.1684 87.0712) (end 129.9972 88.9) (width 0.25) (layer "F.Cu") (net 9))
 (segment (start 118.872 90.489) (end 118.872 90.112928) (width 0.25) (layer "F.Cu") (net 9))
 (segment (start 120.084928 88.9) (end 122.464928 88.9) (width 0.25) (layer "F.Cu") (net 9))
 (segment (start 124.7773 87.0712) (end 128.1684 87.0712) (width 0.25) (layer "F.Cu") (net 9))
 (segment (start 124.775 87.0735) (end 124.7773 87.0712) (width 0.25) (layer "F.Cu") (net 9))
 (segment (start 122.464928 88.9) (end 124.291428 87.0735) (width 0.25) (layer "F.Cu") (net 9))
 (segment (start 118.872 90.112928) (end 120.084928 88.9) (width 0.25) (layer "F.Cu") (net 9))
 (segment (start 128.354598 86.62168) (end 129.362918 87.63) (width 0.25) (layer "F.Cu") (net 10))
 (segment (start 122.875 87.0735) (end 123.93702 86.01148) (width 0.25) (layer "F.Cu") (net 10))
 (segment (start 125.4246 86.01148) (end 126.0348 86.62168) (width 0.25) (layer "F.Cu") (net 10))
 (segment (start 117.602 90.112928) (end 119.576928 88.138) (width 0.25) (layer "F.Cu") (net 10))
 (segment (start 126.0348 86.62168) (end 128.354598 86.62168) (width 0.25) (layer "F.Cu") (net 10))
 (segment (start 117.602 90.489) (end 117.602 90.112928) (width 0.25) (layer "F.Cu") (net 10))
 (segment (start 129.362918 87.63) (end 132.08 87.63) (width 0.25) (layer "F.Cu") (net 10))
 (segment (start 119.576928 88.138) (end 121.8105 88.138) (width 0.25) (layer "F.Cu") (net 10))
 (segment (start 121.8105 88.138) (end 122.875 87.0735) (width 0.25) (layer "F.Cu") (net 10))
 (segment (start 123.93702 86.01148) (end 125.4246 86.01148) (width 0.25) (layer "F.Cu") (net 10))
 (segment (start 112.268 88.456) (end 106.426 94.298) (width 0.25) (layer "F.Cu") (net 4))
 (segment (start 106.108 93.98) (end 102.616 93.98) (width 0.25) (layer "F.Cu") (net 4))
 (segment (start 112.268 87.282) (end 112.268 88.456) (width 0.25) (layer "F.Cu") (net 4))
 (segment (start 106.426 94.298) (end 106.108 93.98) (width 0.25) (layer "F.Cu") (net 4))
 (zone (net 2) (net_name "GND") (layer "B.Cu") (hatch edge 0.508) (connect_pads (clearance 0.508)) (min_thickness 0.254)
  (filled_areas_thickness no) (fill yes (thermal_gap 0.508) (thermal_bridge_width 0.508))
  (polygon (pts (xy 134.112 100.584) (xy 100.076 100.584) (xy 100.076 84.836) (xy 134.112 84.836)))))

